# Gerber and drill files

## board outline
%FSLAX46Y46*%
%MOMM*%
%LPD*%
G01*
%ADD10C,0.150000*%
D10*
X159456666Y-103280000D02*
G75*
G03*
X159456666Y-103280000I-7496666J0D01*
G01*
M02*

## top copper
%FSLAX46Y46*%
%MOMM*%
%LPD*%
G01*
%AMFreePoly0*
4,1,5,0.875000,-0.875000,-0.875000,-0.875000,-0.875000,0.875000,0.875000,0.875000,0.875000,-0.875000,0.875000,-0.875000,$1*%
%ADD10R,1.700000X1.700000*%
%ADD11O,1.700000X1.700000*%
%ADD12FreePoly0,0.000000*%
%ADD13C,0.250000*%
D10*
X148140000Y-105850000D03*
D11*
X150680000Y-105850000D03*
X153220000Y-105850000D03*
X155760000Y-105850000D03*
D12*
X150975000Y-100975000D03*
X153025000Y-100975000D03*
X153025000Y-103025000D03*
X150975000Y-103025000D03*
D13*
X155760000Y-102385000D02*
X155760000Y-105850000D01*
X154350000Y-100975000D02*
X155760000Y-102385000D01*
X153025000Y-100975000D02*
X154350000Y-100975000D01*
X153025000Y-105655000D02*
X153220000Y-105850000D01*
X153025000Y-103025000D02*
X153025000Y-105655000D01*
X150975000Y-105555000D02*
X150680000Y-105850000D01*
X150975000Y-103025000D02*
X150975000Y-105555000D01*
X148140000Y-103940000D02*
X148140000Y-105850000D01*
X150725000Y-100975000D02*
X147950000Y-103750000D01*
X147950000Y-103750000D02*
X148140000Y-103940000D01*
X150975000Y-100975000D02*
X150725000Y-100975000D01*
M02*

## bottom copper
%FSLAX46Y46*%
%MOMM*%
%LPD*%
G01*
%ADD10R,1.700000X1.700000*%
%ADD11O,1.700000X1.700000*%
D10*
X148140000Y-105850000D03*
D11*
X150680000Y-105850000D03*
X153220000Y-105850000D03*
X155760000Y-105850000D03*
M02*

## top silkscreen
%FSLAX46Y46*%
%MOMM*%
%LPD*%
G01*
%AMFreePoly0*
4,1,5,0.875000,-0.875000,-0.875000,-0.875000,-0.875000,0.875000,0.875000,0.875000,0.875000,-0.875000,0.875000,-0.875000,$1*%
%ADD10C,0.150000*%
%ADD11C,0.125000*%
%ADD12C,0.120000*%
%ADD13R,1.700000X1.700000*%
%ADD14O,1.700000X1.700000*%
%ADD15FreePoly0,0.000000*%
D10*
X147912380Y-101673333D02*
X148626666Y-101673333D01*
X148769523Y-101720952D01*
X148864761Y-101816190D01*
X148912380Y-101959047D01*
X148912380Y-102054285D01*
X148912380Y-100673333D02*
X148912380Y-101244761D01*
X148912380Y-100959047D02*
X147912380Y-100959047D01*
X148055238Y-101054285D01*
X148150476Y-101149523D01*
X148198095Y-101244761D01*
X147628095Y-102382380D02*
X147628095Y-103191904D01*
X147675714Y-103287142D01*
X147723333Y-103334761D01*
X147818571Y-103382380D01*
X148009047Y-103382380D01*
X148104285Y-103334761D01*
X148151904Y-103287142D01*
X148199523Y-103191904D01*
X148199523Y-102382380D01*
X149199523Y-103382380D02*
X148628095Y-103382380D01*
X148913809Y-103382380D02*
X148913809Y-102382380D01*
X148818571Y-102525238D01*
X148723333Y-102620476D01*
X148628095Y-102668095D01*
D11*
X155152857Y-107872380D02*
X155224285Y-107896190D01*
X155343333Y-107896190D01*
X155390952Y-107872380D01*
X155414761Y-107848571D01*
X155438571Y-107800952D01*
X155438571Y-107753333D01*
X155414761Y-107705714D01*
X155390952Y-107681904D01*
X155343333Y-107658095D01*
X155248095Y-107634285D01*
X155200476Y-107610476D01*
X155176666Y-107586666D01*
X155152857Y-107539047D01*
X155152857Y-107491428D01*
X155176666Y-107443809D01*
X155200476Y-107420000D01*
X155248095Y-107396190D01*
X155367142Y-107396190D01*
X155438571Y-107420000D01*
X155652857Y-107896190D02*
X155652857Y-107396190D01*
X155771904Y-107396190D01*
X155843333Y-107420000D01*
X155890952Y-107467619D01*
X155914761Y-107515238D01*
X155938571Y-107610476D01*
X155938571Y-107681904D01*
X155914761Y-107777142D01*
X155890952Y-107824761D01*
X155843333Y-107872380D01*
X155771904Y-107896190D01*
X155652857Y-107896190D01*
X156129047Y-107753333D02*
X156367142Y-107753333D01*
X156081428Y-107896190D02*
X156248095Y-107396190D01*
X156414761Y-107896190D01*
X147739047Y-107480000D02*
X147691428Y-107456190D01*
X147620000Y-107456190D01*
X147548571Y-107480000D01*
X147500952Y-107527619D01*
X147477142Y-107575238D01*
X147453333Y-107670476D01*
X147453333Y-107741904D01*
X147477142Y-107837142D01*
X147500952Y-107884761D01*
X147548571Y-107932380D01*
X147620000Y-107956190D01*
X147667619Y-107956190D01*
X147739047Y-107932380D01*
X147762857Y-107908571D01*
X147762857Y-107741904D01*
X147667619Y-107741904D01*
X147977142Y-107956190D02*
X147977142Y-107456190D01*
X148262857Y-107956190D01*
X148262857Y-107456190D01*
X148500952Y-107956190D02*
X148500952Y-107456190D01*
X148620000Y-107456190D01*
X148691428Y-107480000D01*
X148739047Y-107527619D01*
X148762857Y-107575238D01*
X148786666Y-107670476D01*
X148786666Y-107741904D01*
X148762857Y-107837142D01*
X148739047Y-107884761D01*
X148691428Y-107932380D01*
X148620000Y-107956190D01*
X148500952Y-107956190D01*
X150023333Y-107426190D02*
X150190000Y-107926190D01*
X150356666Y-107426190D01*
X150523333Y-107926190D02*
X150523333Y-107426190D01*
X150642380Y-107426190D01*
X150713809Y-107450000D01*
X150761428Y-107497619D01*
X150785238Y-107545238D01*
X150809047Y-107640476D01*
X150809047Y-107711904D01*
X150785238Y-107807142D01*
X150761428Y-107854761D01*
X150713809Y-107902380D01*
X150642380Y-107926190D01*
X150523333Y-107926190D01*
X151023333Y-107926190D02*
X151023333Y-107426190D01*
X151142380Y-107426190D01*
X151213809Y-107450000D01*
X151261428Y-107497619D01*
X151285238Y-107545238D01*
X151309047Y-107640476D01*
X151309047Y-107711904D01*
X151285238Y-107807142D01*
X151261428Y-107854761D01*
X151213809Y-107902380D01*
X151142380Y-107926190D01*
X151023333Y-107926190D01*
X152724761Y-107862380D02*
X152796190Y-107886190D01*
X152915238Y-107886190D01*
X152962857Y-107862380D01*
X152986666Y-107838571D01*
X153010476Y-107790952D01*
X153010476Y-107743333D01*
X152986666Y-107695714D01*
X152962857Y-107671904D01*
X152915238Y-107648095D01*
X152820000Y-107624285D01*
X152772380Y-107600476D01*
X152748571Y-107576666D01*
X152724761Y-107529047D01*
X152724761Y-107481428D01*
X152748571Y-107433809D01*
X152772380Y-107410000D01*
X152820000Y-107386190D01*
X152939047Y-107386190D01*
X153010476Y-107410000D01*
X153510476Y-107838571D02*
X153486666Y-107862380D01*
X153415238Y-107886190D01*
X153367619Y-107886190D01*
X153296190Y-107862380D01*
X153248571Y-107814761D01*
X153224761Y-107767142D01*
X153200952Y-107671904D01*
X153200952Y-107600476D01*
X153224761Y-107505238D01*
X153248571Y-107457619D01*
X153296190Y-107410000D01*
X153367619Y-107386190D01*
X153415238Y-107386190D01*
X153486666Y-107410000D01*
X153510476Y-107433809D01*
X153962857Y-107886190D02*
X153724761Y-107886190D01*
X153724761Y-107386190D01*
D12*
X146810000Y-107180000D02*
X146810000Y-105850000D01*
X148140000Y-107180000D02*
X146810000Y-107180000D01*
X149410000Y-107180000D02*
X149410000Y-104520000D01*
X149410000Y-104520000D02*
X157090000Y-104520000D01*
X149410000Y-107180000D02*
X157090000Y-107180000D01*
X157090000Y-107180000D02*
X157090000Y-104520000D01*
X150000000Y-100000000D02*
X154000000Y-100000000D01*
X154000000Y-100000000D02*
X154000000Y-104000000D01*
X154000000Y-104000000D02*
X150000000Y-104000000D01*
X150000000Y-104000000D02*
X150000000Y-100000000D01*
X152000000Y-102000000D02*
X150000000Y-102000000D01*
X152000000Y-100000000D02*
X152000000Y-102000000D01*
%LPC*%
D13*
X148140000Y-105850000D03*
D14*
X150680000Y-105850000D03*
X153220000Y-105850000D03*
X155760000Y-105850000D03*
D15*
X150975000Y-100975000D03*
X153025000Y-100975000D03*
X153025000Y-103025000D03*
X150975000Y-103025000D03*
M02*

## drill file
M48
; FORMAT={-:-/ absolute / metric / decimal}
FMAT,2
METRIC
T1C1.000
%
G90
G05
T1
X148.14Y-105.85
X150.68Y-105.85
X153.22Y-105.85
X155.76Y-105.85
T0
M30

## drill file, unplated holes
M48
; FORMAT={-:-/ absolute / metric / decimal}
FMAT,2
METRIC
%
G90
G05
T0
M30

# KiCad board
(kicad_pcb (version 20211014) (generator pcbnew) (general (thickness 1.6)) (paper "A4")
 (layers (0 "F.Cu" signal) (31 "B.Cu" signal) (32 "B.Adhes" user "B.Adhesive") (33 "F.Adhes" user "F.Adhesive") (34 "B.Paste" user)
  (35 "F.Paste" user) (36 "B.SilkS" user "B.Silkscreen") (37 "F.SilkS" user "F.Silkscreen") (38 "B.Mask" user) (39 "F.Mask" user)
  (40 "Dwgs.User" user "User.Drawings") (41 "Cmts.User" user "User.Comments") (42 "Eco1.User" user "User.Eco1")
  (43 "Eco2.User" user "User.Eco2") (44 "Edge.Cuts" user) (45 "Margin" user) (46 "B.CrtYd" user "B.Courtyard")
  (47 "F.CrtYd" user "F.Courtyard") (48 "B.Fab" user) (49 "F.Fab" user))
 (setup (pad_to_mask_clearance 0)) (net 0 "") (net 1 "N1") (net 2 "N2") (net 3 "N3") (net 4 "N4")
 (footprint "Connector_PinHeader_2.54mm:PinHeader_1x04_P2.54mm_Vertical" (layer "F.Cu") (at 148.14 105.85 90)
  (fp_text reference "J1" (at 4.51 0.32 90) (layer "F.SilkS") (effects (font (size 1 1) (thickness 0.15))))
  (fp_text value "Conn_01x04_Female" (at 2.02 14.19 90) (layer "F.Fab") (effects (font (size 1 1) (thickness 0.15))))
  (fp_line (start -1.33 -1.33) (end 0 -1.33) (layer "F.SilkS") (width 0.12))
  (fp_line (start -1.33 1.27) (end -1.33 8.95) (layer "F.SilkS") (width 0.12))
  (fp_line (start 1.33 1.27) (end 1.33 8.95) (layer "F.SilkS") (width 0.12))
  (fp_line (start -1.33 1.27) (end 1.33 1.27) (layer "F.SilkS") (width 0.12))
  (fp_line (start -1.33 0) (end -1.33 -1.33) (layer "F.SilkS") (width 0.12))
  (fp_line (start -1.33 8.95) (end 1.33 8.95) (layer "F.SilkS") (width 0.12))
  (pad "1" thru_hole rect locked (at 0 0 90) (size 1.7 1.7) (drill 1) (layers *.Cu *.Mask) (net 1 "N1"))
  (pad "2" thru_hole oval locked (at 0 2.54 90) (size 1.7 1.7) (drill 1) (layers *.Cu *.Mask) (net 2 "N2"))
  (pad "3" thru_hole oval locked (at 0 5.08 90) (size 1.7 1.7) (drill 1) (layers *.Cu *.Mask) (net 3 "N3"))
  (pad "4" thru_hole oval locked (at 0 7.62 90) (size 1.7 1.7) (drill 1) (layers *.Cu *.Mask) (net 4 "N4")))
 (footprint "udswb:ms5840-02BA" (layer "F.Cu") (at 150 100)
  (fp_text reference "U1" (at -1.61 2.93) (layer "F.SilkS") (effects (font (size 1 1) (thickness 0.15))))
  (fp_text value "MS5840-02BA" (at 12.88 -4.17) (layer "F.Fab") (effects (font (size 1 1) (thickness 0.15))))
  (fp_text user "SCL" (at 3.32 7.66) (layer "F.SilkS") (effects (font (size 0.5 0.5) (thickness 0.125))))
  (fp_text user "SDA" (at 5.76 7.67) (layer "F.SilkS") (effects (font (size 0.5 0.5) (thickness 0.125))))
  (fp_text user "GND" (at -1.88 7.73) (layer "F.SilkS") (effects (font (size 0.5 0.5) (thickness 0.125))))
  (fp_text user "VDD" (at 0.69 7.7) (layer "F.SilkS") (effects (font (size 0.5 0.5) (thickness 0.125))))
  (fp_line (start 0 4) (end 0 0) (layer "F.SilkS") (width 0.12))
  (fp_line (start 4 0) (end 4 4) (layer "F.SilkS") (width 0.12))
  (fp_line (start 0 0) (end 4 0) (layer "F.SilkS") (width 0.12))
  (fp_line (start 2 2) (end 0 2) (layer "F.SilkS") (width 0.12))
  (fp_line (start 4 4) (end 0 4) (layer "F.SilkS") (width 0.12))
  (fp_line (start 2 0) (end 2 2) (layer "F.SilkS") (width 0.12))
  (pad "1" smd custom locked (at 0.975 0.975) (size 1.75 1.75) (layers "F.Cu" "F.Paste" "F.Mask") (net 1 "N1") (zone_connect 0)
   (options (clearance outline) (anchor rect)) (primitives))
  (pad "2" smd custom locked (at 0.975 3.025) (size 1.75 1.75) (layers "F.Cu" "F.Paste" "F.Mask") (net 2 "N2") (zone_connect 0)
   (options (clearance outline) (anchor rect)) (primitives))
  (pad "3" smd custom locked (at 3.025 3.025) (size 1.75 1.75) (layers "F.Cu" "F.Paste" "F.Mask") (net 3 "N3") (zone_connect 0)
   (options (clearance outline) (anchor rect)) (primitives))
  (pad "4" smd custom locked (at 3.025 0.975) (size 1.75 1.75) (layers "F.Cu" "F.Paste" "F.Mask") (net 4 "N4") (zone_connect 0)
   (options (clearance outline) (anchor rect)) (primitives)))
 (gr_circle (center 151.96 103.28) (end 159.456666 103.28) (layer "Edge.Cuts") (width 0.15) (fill none))
 (segment (start 150.725 100.975) (end 147.95 103.75) (width 0.25) (layer "F.Cu") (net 1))
 (segment (start 147.95 103.75) (end 148.14 103.94) (width 0.25) (layer "F.Cu") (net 1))
 (segment (start 148.14 103.94) (end 148.14 105.85) (width 0.25) (layer "F.Cu") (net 1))
 (segment (start 150.975 100.975) (end 150.725 100.975) (width 0.25) (layer "F.Cu") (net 1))
 (segment (start 150.975 105.555) (end 150.68 105.85) (width 0.25) (layer "F.Cu") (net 2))
 (segment (start 150.975 103.025) (end 150.975 105.555) (width 0.25) (layer "F.Cu") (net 2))
 (segment (start 153.025 105.655) (end 153.22 105.85) (width 0.25) (layer "F.Cu") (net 3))
 (segment (start 153.025 103.025) (end 153.025 105.655) (width 0.25) (layer "F.Cu") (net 3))
 (segment (start 154.35 100.975) (end 155.76 102.385) (width 0.25) (layer "F.Cu") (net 4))
 (segment (start 155.76 102.385) (end 155.76 105.85) (width 0.25) (layer "F.Cu") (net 4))
 (segment (start 153.025 100.975) (end 154.35 100.975) (width 0.25) (layer "F.Cu") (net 4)))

